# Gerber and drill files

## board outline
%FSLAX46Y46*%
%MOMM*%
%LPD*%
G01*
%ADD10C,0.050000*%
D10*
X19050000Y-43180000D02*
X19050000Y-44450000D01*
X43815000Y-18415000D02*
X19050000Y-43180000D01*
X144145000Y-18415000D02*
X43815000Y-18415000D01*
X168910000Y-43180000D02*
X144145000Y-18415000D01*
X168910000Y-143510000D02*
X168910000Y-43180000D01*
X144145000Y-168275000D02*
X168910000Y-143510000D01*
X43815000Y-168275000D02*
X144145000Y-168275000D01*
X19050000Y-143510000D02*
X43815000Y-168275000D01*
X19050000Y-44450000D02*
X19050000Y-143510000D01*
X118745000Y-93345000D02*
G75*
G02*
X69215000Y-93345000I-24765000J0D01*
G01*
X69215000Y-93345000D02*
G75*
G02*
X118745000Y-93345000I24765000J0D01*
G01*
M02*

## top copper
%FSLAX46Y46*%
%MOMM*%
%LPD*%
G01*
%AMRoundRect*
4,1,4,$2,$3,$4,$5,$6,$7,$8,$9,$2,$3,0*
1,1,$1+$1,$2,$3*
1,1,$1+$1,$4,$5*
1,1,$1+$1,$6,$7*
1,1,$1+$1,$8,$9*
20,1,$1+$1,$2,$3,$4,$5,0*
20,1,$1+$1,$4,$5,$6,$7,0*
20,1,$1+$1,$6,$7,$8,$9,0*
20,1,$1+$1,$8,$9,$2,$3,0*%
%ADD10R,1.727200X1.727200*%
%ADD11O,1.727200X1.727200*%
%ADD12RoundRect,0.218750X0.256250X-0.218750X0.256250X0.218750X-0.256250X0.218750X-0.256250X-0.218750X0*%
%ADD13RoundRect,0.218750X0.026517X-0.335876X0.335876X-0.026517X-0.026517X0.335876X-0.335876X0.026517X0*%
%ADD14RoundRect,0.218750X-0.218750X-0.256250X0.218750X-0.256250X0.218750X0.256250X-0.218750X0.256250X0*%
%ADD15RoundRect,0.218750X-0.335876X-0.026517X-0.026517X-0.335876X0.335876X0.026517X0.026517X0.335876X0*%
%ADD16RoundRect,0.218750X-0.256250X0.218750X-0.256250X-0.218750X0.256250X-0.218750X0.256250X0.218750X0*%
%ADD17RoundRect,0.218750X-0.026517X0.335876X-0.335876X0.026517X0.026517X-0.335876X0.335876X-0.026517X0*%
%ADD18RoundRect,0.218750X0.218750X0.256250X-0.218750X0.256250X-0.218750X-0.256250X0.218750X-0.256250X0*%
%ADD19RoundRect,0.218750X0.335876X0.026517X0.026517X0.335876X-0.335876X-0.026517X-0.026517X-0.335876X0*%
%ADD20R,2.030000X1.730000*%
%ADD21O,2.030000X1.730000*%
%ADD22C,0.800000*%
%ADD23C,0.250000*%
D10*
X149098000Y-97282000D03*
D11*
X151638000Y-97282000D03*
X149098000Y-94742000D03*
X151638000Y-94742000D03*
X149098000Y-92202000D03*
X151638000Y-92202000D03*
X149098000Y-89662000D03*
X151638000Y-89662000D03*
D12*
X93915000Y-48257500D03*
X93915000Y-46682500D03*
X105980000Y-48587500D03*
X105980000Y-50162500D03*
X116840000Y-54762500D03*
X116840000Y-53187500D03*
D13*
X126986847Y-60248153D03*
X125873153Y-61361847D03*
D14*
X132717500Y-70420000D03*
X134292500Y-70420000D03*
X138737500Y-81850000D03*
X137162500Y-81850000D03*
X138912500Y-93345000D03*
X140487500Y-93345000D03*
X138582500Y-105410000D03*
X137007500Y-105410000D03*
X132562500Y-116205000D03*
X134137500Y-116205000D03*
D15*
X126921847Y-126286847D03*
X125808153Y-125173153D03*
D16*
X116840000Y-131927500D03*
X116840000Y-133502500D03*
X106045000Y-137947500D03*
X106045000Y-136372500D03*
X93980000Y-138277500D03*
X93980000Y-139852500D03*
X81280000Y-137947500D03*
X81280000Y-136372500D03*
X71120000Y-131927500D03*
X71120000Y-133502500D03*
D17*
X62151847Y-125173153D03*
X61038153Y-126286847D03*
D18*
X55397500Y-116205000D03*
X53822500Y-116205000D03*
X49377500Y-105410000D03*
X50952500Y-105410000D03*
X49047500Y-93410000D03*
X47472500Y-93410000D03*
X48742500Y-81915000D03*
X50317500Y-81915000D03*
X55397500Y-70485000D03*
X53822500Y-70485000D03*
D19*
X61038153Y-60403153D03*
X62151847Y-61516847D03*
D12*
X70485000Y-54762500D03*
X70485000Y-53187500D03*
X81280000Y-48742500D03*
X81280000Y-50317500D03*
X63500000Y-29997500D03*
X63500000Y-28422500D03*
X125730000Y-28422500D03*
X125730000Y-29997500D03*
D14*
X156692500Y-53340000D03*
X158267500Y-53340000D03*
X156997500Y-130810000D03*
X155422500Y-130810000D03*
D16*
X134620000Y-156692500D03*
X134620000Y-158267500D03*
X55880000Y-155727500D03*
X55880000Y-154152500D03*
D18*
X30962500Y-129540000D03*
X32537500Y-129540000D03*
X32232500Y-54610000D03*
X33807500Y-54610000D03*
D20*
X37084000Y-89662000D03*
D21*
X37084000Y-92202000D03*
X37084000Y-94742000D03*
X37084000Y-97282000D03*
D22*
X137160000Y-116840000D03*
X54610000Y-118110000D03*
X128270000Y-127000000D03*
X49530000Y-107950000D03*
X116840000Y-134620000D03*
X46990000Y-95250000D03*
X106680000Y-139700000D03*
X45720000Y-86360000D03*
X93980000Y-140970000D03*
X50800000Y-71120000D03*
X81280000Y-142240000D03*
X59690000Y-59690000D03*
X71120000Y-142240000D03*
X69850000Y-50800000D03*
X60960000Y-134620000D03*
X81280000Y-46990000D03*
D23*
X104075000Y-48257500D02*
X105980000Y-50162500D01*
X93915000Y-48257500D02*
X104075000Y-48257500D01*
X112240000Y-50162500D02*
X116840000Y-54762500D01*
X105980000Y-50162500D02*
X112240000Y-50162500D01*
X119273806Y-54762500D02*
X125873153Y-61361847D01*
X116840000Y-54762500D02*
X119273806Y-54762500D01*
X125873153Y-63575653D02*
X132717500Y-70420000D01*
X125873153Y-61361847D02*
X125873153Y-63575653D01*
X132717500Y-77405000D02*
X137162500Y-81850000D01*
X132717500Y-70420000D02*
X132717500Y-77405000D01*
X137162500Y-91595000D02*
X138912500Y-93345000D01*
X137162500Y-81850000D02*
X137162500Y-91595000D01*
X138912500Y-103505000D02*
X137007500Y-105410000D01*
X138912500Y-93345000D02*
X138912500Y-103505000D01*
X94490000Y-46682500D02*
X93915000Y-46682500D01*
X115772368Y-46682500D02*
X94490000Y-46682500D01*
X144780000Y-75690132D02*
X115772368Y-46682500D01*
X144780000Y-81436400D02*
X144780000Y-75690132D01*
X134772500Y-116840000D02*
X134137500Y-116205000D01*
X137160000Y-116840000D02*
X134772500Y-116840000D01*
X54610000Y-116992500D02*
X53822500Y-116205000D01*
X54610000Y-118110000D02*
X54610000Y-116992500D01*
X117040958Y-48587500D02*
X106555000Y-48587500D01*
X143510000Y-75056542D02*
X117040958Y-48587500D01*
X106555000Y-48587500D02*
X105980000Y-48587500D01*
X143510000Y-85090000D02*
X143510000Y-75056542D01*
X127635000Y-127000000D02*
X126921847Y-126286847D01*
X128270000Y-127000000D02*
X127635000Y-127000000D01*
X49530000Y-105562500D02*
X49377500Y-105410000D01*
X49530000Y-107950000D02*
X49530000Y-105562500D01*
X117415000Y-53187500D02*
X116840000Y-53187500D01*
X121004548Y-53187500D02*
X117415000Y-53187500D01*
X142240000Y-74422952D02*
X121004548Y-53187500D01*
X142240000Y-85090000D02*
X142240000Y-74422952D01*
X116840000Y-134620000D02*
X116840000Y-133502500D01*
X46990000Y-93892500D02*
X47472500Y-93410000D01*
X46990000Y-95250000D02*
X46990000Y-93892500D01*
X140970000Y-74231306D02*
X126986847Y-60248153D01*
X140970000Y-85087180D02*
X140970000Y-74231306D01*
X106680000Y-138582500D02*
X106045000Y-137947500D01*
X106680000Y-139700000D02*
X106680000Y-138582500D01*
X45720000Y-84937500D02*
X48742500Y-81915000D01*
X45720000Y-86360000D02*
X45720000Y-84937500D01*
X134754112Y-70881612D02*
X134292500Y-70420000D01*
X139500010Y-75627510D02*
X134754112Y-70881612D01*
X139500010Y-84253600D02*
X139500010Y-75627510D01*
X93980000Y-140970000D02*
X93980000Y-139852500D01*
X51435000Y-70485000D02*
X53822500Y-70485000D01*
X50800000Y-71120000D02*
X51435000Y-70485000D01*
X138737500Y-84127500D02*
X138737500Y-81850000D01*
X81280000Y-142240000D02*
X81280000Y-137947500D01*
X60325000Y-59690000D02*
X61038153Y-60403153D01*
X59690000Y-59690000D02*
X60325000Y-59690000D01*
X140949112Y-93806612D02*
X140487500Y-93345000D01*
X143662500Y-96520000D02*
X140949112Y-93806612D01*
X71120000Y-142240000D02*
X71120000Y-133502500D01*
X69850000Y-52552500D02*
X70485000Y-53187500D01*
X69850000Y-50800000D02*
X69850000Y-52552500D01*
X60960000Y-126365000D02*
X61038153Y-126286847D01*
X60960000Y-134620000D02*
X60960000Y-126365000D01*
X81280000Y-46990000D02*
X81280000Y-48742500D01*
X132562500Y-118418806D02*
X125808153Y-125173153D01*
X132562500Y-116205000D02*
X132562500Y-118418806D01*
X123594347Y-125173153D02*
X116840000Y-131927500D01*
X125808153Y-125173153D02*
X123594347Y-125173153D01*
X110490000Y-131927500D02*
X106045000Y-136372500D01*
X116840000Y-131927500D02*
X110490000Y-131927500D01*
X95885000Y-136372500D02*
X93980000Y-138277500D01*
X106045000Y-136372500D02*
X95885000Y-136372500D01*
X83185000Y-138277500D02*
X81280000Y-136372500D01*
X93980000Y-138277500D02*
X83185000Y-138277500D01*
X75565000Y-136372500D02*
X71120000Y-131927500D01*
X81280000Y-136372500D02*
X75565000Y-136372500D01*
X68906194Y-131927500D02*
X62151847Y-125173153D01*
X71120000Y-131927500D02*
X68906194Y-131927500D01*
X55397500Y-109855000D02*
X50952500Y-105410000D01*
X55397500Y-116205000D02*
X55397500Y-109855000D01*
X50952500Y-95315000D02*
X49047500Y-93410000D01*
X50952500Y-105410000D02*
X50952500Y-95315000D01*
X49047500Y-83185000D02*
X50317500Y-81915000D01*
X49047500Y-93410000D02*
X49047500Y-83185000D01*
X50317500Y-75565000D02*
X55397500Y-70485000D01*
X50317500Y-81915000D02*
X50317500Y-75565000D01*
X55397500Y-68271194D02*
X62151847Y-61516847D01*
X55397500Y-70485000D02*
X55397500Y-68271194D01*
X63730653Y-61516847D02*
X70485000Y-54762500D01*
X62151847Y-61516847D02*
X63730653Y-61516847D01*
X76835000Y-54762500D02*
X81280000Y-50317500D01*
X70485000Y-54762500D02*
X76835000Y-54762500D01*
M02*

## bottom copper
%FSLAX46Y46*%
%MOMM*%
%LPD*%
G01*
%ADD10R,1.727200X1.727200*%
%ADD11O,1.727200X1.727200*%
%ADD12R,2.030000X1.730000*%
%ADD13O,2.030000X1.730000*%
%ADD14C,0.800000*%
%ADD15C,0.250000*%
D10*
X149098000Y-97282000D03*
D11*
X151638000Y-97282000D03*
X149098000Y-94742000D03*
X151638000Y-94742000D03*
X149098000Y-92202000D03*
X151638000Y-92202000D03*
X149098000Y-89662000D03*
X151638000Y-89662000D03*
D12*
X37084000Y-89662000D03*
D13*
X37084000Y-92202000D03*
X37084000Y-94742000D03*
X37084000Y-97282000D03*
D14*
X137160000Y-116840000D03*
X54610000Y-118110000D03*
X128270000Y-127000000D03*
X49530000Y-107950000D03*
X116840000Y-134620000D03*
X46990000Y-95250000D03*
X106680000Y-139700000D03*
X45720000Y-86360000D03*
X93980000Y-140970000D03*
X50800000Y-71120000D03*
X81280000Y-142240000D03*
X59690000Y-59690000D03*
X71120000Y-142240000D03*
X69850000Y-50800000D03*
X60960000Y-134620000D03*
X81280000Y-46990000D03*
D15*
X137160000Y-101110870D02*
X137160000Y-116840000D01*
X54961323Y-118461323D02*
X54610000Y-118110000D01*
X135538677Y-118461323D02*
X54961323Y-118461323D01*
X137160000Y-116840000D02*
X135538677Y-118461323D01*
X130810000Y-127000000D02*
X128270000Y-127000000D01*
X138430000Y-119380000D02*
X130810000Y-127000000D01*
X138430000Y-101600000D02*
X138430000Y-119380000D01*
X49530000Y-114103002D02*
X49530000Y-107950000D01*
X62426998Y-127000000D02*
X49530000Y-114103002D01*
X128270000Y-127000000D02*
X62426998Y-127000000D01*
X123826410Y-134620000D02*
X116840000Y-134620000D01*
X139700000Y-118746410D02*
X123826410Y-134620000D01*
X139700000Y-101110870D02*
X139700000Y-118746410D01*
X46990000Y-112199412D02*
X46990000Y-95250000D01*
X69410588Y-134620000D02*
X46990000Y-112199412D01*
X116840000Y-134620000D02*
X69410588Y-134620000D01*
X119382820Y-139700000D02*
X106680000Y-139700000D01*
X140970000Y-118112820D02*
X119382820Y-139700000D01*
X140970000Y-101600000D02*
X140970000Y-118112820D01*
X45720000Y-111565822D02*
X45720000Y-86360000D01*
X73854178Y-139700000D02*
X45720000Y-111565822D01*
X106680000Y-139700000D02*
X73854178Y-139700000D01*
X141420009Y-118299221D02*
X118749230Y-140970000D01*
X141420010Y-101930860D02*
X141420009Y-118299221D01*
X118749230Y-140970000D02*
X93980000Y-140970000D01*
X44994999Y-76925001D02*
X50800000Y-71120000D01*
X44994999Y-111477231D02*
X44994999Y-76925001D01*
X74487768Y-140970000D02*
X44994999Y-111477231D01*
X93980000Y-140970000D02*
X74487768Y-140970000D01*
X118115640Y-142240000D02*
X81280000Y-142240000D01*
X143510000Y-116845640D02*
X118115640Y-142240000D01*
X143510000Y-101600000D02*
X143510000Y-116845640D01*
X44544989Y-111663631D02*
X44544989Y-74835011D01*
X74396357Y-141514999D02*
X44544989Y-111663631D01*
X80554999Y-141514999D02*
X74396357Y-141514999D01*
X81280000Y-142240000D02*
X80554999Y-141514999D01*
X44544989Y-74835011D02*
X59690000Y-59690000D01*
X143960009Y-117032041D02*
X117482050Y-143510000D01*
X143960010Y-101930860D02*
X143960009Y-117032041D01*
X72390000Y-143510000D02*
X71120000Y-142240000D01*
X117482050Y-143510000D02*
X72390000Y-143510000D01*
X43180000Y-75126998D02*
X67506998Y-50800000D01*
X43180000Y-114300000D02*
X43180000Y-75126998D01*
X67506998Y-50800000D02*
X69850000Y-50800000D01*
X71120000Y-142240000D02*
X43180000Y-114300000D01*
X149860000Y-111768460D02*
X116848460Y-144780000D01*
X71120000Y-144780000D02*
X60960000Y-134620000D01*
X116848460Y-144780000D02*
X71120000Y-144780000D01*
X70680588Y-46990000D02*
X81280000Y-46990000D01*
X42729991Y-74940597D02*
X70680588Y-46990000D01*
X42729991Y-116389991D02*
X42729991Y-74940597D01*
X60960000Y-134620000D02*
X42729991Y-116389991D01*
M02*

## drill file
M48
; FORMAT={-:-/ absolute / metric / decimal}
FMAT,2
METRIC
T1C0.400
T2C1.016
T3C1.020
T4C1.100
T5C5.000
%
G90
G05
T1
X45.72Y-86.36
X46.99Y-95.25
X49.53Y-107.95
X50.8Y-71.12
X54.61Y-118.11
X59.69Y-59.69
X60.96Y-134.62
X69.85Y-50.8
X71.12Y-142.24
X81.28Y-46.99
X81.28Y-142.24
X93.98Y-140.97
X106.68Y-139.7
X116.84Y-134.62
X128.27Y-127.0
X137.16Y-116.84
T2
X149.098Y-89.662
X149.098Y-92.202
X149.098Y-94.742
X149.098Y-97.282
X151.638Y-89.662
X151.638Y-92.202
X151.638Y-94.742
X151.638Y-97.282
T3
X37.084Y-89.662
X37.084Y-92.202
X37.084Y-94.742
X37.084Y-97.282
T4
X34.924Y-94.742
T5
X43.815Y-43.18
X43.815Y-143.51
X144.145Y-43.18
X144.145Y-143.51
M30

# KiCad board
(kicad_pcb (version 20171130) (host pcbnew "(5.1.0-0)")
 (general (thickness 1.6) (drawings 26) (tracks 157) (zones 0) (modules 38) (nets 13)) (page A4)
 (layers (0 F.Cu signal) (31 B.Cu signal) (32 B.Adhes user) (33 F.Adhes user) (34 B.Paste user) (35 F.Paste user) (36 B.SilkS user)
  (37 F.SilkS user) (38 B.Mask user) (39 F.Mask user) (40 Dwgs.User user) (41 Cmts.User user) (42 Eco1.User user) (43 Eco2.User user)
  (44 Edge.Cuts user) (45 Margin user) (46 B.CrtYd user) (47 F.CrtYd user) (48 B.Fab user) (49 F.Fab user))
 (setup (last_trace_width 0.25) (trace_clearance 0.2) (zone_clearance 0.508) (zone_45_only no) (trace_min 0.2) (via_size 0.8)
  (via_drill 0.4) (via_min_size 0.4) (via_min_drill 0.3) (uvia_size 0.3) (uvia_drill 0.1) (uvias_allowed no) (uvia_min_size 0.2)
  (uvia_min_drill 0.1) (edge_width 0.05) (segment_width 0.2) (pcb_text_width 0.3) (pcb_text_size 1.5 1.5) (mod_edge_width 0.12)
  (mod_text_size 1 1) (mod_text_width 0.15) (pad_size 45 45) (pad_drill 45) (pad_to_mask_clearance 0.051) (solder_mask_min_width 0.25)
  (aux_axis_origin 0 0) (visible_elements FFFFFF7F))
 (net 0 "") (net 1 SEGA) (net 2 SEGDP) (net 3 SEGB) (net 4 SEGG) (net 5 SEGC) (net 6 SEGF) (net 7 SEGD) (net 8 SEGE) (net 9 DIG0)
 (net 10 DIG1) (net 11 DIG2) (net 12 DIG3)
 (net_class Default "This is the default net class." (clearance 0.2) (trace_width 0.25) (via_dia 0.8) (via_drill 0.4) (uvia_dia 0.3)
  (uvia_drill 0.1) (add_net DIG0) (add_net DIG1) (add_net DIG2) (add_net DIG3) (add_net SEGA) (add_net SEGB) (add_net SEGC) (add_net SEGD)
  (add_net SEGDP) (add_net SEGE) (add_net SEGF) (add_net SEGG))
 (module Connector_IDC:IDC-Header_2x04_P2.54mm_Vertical (layer B.Cu) (at 149.098 97.282)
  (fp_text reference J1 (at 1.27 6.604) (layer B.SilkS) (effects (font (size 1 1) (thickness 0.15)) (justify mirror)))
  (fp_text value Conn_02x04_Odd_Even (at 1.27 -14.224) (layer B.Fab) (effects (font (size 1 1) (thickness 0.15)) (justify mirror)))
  (pad 1 thru_hole rect (at 0 0) (size 1.7272 1.7272) (drill 1.016) (layers *.Cu *.Mask) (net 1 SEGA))
  (pad 2 thru_hole oval (at 2.54 0) (size 1.7272 1.7272) (drill 1.016) (layers *.Cu *.Mask) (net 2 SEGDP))
  (pad 3 thru_hole oval (at 0 -2.54) (size 1.7272 1.7272) (drill 1.016) (layers *.Cu *.Mask) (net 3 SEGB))
  (pad 4 thru_hole oval (at 2.54 -2.54) (size 1.7272 1.7272) (drill 1.016) (layers *.Cu *.Mask) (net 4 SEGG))
  (pad 5 thru_hole oval (at 0 -5.08) (size 1.7272 1.7272) (drill 1.016) (layers *.Cu *.Mask) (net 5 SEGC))
  (pad 6 thru_hole oval (at 2.54 -5.08) (size 1.7272 1.7272) (drill 1.016) (layers *.Cu *.Mask) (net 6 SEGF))
  (pad 7 thru_hole oval (at 0 -7.62) (size 1.7272 1.7272) (drill 1.016) (layers *.Cu *.Mask) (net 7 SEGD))
  (pad 8 thru_hole oval (at 2.54 -7.62) (size 1.7272 1.7272) (drill 1.016) (layers *.Cu *.Mask) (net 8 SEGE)))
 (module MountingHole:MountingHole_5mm (layer F.Cu) (at 144.145 43.18)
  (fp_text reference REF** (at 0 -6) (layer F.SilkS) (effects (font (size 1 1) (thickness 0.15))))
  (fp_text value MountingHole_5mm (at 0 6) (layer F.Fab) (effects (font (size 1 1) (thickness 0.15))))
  (pad 1 np_thru_hole circle (at 0 0) (size 5 5) (drill 5) (layers *.Cu *.Mask)))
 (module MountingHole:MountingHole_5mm (layer F.Cu) (at 43.815 43.18)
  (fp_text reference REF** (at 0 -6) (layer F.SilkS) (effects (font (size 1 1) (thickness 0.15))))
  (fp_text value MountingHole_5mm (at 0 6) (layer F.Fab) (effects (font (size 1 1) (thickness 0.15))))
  (pad 1 np_thru_hole circle (at 0 0) (size 5 5) (drill 5) (layers *.Cu *.Mask)))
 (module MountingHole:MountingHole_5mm (layer F.Cu) (at 43.815 143.51)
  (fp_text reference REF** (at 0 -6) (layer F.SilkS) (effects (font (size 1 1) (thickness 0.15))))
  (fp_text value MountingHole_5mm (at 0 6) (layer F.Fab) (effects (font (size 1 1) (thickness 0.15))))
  (pad 1 np_thru_hole circle (at 0 0) (size 5 5) (drill 5) (layers *.Cu *.Mask)))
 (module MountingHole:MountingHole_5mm (layer F.Cu) (at 144.145 143.51)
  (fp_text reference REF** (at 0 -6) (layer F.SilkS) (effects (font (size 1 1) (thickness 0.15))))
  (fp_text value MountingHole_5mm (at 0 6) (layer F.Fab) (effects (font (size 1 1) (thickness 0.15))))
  (pad 1 np_thru_hole circle (at 0 0) (size 5 5) (drill 5) (layers *.Cu *.Mask)))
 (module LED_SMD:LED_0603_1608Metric (layer F.Cu) (at 93.915 47.47 90)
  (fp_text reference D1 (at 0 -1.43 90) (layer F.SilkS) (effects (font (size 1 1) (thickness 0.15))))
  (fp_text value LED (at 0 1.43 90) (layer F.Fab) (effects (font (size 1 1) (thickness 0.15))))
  (pad 1 smd roundrect (at -0.7875 0 90) (size 0.875 0.95) (layers F.Cu F.Paste F.Mask) (roundrect_rratio 0.25) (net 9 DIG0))
  (pad 2 smd roundrect (at 0.7875 0 90) (size 0.875 0.95) (layers F.Cu F.Paste F.Mask) (roundrect_rratio 0.25) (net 1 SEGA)))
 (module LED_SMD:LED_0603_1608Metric (layer F.Cu) (at 105.98 49.375 90)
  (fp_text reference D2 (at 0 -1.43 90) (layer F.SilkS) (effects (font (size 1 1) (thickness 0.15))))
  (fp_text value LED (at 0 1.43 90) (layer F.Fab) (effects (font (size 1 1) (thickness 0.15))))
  (pad 2 smd roundrect (at 0.7875 0 90) (size 0.875 0.95) (layers F.Cu F.Paste F.Mask) (roundrect_rratio 0.25) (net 3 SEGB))
  (pad 1 smd roundrect (at -0.7875 0 90) (size 0.875 0.95) (layers F.Cu F.Paste F.Mask) (roundrect_rratio 0.25) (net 9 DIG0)))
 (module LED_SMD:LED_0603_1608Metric (layer F.Cu) (at 116.84 53.975 90)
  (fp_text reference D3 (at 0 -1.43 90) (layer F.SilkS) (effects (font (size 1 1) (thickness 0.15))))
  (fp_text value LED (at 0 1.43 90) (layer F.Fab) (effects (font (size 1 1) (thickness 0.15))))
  (pad 1 smd roundrect (at -0.7875 0 90) (size 0.875 0.95) (layers F.Cu F.Paste F.Mask) (roundrect_rratio 0.25) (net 9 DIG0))
  (pad 2 smd roundrect (at 0.7875 0 90) (size 0.875 0.95) (layers F.Cu F.Paste F.Mask) (roundrect_rratio 0.25) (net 5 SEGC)))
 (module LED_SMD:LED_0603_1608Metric (layer F.Cu) (at 126.43 60.805 45)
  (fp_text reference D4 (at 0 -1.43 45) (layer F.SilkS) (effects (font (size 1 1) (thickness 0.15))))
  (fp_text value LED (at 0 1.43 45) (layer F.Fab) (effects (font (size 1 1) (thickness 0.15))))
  (pad 2 smd roundrect (at 0.7875 0 45) (size 0.875 0.95) (layers F.Cu F.Paste F.Mask) (roundrect_rratio 0.25) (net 7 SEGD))
  (pad 1 smd roundrect (at -0.7875 0 45) (size 0.875 0.95) (layers F.Cu F.Paste F.Mask) (roundrect_rratio 0.25) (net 9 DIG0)))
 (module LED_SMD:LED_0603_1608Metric (layer F.Cu) (at 133.505 70.42)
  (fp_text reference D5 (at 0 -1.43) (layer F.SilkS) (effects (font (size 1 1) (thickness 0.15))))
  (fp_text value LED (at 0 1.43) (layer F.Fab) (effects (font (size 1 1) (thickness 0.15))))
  (pad 1 smd roundrect (at -0.7875 0) (size 0.875 0.95) (layers F.Cu F.Paste F.Mask) (roundrect_rratio 0.25) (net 9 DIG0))
  (pad 2 smd roundrect (at 0.7875 0) (size 0.875 0.95) (layers F.Cu F.Paste F.Mask) (roundrect_rratio 0.25) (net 8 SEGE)))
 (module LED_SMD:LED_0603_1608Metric (layer F.Cu) (at 137.95 81.85)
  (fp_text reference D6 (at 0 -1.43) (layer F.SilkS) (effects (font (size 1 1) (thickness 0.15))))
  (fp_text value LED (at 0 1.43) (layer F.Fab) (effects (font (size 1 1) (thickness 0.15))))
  (pad 2 smd roundrect (at 0.7875 0) (size 0.875 0.95) (layers F.Cu F.Paste F.Mask) (roundrect_rratio 0.25) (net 6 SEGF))
  (pad 1 smd roundrect (at -0.7875 0) (size 0.875 0.95) (layers F.Cu F.Paste F.Mask) (roundrect_rratio 0.25) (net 9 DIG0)))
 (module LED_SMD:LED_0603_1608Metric (layer F.Cu) (at 139.7 93.345)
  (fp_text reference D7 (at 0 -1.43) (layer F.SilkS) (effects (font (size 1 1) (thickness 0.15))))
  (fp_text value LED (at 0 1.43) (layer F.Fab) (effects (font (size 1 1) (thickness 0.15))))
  (pad 1 smd roundrect (at -0.7875 0) (size 0.875 0.95) (layers F.Cu F.Paste F.Mask) (roundrect_rratio 0.25) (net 9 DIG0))
  (pad 2 smd roundrect (at 0.7875 0) (size 0.875 0.95) (layers F.Cu F.Paste F.Mask) (roundrect_rratio 0.25) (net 4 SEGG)))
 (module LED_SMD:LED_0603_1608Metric (layer F.Cu) (at 137.795 105.41)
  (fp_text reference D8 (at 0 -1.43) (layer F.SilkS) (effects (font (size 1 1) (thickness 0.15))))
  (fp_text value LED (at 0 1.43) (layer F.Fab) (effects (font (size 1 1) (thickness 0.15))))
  (pad 2 smd roundrect (at 0.7875 0) (size 0.875 0.95) (layers F.Cu F.Paste F.Mask) (roundrect_rratio 0.25) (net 2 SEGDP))
  (pad 1 smd roundrect (at -0.7875 0) (size 0.875 0.95) (layers F.Cu F.Paste F.Mask) (roundrect_rratio 0.25) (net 9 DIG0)))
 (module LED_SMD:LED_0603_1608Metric (layer F.Cu) (at 133.35 116.205)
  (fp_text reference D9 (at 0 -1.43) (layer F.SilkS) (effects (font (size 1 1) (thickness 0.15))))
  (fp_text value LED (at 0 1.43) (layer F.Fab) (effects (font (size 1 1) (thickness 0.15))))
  (pad 1 smd roundrect (at -0.7875 0) (size 0.875 0.95) (layers F.Cu F.Paste F.Mask) (roundrect_rratio 0.25) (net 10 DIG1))
  (pad 2 smd roundrect (at 0.7875 0) (size 0.875 0.95) (layers F.Cu F.Paste F.Mask) (roundrect_rratio 0.25) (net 1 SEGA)))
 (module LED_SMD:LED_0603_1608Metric (layer F.Cu) (at 126.365 125.73 315)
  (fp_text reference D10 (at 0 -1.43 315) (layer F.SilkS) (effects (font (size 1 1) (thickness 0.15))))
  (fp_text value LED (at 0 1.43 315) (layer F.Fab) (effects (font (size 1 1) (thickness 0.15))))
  (pad 2 smd roundrect (at 0.7875 0 315) (size 0.875 0.95) (layers F.Cu F.Paste F.Mask) (roundrect_rratio 0.25) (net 3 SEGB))
  (pad 1 smd roundrect (at -0.7875 0 315) (size 0.875 0.95) (layers F.Cu F.Paste F.Mask) (roundrect_rratio 0.25) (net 10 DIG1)))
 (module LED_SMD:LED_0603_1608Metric (layer F.Cu) (at 116.84 132.715 270)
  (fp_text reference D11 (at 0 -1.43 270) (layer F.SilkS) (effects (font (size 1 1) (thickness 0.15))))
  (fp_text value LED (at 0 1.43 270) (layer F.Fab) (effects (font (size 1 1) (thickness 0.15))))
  (pad 1 smd roundrect (at -0.7875 0 270) (size 0.875 0.95) (layers F.Cu F.Paste F.Mask) (roundrect_rratio 0.25) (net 10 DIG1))
  (pad 2 smd roundrect (at 0.7875 0 270) (size 0.875 0.95) (layers F.Cu F.Paste F.Mask) (roundrect_rratio 0.25) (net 5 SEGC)))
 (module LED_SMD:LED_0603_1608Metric (layer F.Cu) (at 106.045 137.16 270)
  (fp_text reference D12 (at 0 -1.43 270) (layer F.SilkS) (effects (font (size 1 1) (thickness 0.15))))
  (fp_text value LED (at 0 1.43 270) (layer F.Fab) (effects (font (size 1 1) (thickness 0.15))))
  (pad 2 smd roundrect (at 0.7875 0 270) (size 0.875 0.95) (layers F.Cu F.Paste F.Mask) (roundrect_rratio 0.25) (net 7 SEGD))
  (pad 1 smd roundrect (at -0.7875 0 270) (size 0.875 0.95) (layers F.Cu F.Paste F.Mask) (roundrect_rratio 0.25) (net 10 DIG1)))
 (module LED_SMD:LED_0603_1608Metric (layer F.Cu) (at 93.98 139.065 270)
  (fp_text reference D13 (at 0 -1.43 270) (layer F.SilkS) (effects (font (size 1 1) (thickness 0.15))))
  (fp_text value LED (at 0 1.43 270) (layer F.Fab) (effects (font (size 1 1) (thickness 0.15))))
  (pad 1 smd roundrect (at -0.7875 0 270) (size 0.875 0.95) (layers F.Cu F.Paste F.Mask) (roundrect_rratio 0.25) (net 10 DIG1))
  (pad 2 smd roundrect (at 0.7875 0 270) (size 0.875 0.95) (layers F.Cu F.Paste F.Mask) (roundrect_rratio 0.25) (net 8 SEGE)))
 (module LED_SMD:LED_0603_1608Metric (layer F.Cu) (at 81.28 137.16 270)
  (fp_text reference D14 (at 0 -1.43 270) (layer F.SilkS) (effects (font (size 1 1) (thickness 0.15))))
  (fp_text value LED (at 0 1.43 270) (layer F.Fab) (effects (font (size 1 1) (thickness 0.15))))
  (pad 2 smd roundrect (at 0.7875 0 270) (size 0.875 0.95) (layers F.Cu F.Paste F.Mask) (roundrect_rratio 0.25) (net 6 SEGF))
  (pad 1 smd roundrect (at -0.7875 0 270) (size 0.875 0.95) (layers F.Cu F.Paste F.Mask) (roundrect_rratio 0.25) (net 10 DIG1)))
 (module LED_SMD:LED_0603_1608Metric (layer F.Cu) (at 71.12 132.715 270)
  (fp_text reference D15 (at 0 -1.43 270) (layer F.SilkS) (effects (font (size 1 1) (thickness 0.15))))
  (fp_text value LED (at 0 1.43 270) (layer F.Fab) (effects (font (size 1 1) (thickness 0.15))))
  (pad 1 smd roundrect (at -0.7875 0 270) (size 0.875 0.95) (layers F.Cu F.Paste F.Mask) (roundrect_rratio 0.25) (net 10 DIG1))
  (pad 2 smd roundrect (at 0.7875 0 270) (size 0.875 0.95) (layers F.Cu F.Paste F.Mask) (roundrect_rratio 0.25) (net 4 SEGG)))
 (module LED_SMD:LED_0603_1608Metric (layer F.Cu) (at 61.595 125.73 225)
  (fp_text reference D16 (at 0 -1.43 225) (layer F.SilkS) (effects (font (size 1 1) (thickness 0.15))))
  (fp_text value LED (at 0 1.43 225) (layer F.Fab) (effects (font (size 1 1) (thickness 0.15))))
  (pad 1 smd roundrect (at -0.7875 0 225) (size 0.875 0.95) (layers F.Cu F.Paste F.Mask) (roundrect_rratio 0.25) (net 10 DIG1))
  (pad 2 smd roundrect (at 0.7875 0 225) (size 0.875 0.95) (layers F.Cu F.Paste F.Mask) (roundrect_rratio 0.25) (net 2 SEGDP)))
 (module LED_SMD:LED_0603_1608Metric (layer F.Cu) (at 54.61 116.205 180)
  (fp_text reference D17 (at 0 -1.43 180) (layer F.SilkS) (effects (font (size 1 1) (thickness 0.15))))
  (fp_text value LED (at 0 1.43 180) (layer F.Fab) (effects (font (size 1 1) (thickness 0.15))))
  (pad 1 smd roundrect (at -0.7875 0 180) (size 0.875 0.95) (layers F.Cu F.Paste F.Mask) (roundrect_rratio 0.25) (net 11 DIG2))
  (pad 2 smd roundrect (at 0.7875 0 180) (size 0.875 0.95) (layers F.Cu F.Paste F.Mask) (roundrect_rratio 0.25) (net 1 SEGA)))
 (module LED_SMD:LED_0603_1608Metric (layer F.Cu) (at 50.165 105.41 180)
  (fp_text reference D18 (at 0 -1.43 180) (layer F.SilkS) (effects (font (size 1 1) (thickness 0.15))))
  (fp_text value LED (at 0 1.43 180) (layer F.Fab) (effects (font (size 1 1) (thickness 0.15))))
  (pad 2 smd roundrect (at 0.7875 0 180) (size 0.875 0.95) (layers F.Cu F.Paste F.Mask) (roundrect_rratio 0.25) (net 3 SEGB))
  (pad 1 smd roundrect (at -0.7875 0 180) (size 0.875 0.95) (layers F.Cu F.Paste F.Mask) (roundrect_rratio 0.25) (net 11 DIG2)))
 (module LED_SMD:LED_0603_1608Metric (layer F.Cu) (at 48.26 93.41 180)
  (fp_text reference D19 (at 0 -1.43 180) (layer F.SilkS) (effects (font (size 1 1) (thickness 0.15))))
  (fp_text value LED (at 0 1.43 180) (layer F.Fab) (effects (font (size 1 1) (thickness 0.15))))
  (pad 1 smd roundrect (at -0.7875 0 180) (size 0.875 0.95) (layers F.Cu F.Paste F.Mask) (roundrect_rratio 0.25) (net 11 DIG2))
  (pad 2 smd roundrect (at 0.7875 0 180) (size 0.875 0.95) (layers F.Cu F.Paste F.Mask) (roundrect_rratio 0.25) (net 5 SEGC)))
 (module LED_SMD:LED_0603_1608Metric (layer F.Cu) (at 49.53 81.915 180)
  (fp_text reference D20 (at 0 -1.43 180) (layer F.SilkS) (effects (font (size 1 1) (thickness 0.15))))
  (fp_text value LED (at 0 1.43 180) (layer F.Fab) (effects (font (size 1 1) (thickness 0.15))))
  (pad 2 smd roundrect (at 0.7875 0 180) (size 0.875 0.95) (layers F.Cu F.Paste F.Mask) (roundrect_rratio 0.25) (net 7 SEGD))
  (pad 1 smd roundrect (at -0.7875 0 180) (size 0.875 0.95) (layers F.Cu F.Paste F.Mask) (roundrect_rratio 0.25) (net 11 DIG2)))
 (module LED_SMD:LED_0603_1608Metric (layer F.Cu) (at 54.61 70.485 180)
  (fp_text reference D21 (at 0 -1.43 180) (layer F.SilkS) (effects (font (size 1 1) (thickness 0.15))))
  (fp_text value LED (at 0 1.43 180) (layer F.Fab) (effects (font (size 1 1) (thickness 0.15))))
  (pad 1 smd roundrect (at -0.7875 0 180) (size 0.875 0.95) (layers F.Cu F.Paste F.Mask) (roundrect_rratio 0.25) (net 11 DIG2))
  (pad 2 smd roundrect (at 0.7875 0 180) (size 0.875 0.95) (layers F.Cu F.Paste F.Mask) (roundrect_rratio 0.25) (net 8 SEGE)))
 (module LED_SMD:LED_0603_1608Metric (layer F.Cu) (at 61.595 60.96 135)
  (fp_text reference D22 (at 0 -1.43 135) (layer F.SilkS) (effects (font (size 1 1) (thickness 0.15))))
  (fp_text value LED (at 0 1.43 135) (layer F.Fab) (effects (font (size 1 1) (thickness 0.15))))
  (pad 2 smd roundrect (at 0.7875 0 135) (size 0.875 0.95) (layers F.Cu F.Paste F.Mask) (roundrect_rratio 0.25) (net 6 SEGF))
  (pad 1 smd roundrect (at -0.7875 0 135) (size 0.875 0.95) (layers F.Cu F.Paste F.Mask) (roundrect_rratio 0.25) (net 11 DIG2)))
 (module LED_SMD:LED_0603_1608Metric (layer F.Cu) (at 70.485 53.975 90)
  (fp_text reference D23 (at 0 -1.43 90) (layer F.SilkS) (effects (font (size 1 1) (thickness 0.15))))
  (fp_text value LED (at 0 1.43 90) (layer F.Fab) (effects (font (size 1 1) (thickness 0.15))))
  (pad 1 smd roundrect (at -0.7875 0 90) (size 0.875 0.95) (layers F.Cu F.Paste F.Mask) (roundrect_rratio 0.25) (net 11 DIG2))
  (pad 2 smd roundrect (at 0.7875 0 90) (size 0.875 0.95) (layers F.Cu F.Paste F.Mask) (roundrect_rratio 0.25) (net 4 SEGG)))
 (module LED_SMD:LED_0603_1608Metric (layer F.Cu) (at 81.28 49.53 90)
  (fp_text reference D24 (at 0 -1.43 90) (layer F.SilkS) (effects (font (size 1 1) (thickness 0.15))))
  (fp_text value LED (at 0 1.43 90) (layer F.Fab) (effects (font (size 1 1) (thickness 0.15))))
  (pad 2 smd roundrect (at 0.7875 0 90) (size 0.875 0.95) (layers F.Cu F.Paste F.Mask) (roundrect_rratio 0.25) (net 2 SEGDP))
  (pad 1 smd roundrect (at -0.7875 0 90) (size 0.875 0.95) (layers F.Cu F.Paste F.Mask) (roundrect_rratio 0.25) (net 11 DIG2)))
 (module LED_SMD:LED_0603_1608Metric (layer F.Cu) (at 63.5 29.21 90)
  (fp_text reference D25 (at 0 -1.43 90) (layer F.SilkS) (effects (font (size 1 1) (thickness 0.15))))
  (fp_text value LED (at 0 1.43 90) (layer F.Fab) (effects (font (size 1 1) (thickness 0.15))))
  (pad 1 smd roundrect (at -0.7875 0 90) (size 0.875 0.95) (layers F.Cu F.Paste F.Mask) (roundrect_rratio 0.25) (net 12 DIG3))
  (pad 2 smd roundrect (at 0.7875 0 90) (size 0.875 0.95) (layers F.Cu F.Paste F.Mask) (roundrect_rratio 0.25) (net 1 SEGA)))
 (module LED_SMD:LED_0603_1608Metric (layer F.Cu) (at 125.73 29.21 90)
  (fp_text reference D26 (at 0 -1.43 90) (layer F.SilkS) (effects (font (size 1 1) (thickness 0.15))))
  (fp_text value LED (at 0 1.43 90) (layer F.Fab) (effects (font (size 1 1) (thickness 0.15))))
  (pad 2 smd roundrect (at 0.7875 0 90) (size 0.875 0.95) (layers F.Cu F.Paste F.Mask) (roundrect_rratio 0.25) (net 3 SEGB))
  (pad 1 smd roundrect (at -0.7875 0 90) (size 0.875 0.95) (layers F.Cu F.Paste F.Mask) (roundrect_rratio 0.25) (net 12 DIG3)))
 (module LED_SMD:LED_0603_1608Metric (layer F.Cu) (at 157.48 53.34)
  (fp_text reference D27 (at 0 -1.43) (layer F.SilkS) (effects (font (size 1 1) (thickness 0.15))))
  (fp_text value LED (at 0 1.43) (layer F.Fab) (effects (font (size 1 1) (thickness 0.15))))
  (pad 1 smd roundrect (at -0.7875 0) (size 0.875 0.95) (layers F.Cu F.Paste F.Mask) (roundrect_rratio 0.25) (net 12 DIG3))
  (pad 2 smd roundrect (at 0.7875 0) (size 0.875 0.95) (layers F.Cu F.Paste F.Mask) (roundrect_rratio 0.25) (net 5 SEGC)))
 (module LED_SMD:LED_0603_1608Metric (layer F.Cu) (at 156.21 130.81)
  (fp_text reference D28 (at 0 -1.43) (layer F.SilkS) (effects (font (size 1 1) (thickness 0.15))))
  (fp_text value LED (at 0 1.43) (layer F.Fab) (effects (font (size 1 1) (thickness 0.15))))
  (pad 2 smd roundrect (at 0.7875 0) (size 0.875 0.95) (layers F.Cu F.Paste F.Mask) (roundrect_rratio 0.25) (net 7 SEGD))
  (pad 1 smd roundrect (at -0.7875 0) (size 0.875 0.95) (layers F.Cu F.Paste F.Mask) (roundrect_rratio 0.25) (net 12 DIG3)))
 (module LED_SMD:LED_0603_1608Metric (layer F.Cu) (at 134.62 157.48 270)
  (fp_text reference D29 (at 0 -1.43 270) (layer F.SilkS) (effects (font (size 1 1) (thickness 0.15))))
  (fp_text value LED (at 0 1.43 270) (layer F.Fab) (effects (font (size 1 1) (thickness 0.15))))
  (pad 1 smd roundrect (at -0.7875 0 270) (size 0.875 0.95) (layers F.Cu F.Paste F.Mask) (roundrect_rratio 0.25) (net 12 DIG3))
  (pad 2 smd roundrect (at 0.7875 0 270) (size 0.875 0.95) (layers F.Cu F.Paste F.Mask) (roundrect_rratio 0.25) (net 8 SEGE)))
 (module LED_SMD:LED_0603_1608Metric (layer F.Cu) (at 55.88 154.94 270)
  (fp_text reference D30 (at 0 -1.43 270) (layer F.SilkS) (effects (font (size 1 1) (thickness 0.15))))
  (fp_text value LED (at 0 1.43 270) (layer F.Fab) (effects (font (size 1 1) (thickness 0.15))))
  (pad 2 smd roundrect (at 0.7875 0 270) (size 0.875 0.95) (layers F.Cu F.Paste F.Mask) (roundrect_rratio 0.25) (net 6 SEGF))
  (pad 1 smd roundrect (at -0.7875 0 270) (size 0.875 0.95) (layers F.Cu F.Paste F.Mask) (roundrect_rratio 0.25) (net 12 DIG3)))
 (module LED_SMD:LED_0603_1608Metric (layer F.Cu) (at 31.75 129.54 180)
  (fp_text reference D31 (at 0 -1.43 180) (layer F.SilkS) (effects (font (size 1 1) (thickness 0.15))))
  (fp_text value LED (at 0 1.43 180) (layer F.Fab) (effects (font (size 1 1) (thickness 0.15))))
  (pad 2 smd roundrect (at 0.7875 0 180) (size 0.875 0.95) (layers F.Cu F.Paste F.Mask) (roundrect_rratio 0.25) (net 4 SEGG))
  (pad 1 smd roundrect (at -0.7875 0 180) (size 0.875 0.95) (layers F.Cu F.Paste F.Mask) (roundrect_rratio 0.25) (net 12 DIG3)))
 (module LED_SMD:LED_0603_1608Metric (layer F.Cu) (at 33.02 54.61 180)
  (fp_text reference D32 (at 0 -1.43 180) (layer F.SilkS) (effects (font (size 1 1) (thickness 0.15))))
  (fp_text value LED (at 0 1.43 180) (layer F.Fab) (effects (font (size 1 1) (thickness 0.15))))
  (pad 2 smd roundrect (at 0.7875 0 180) (size 0.875 0.95) (layers F.Cu F.Paste F.Mask) (roundrect_rratio 0.25) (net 2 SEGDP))
  (pad 1 smd roundrect (at -0.7875 0 180) (size 0.875 0.95) (layers F.Cu F.Paste F.Mask) (roundrect_rratio 0.25) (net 12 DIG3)))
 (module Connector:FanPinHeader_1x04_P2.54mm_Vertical (layer B.Cu) (at 37.084 89.662 270)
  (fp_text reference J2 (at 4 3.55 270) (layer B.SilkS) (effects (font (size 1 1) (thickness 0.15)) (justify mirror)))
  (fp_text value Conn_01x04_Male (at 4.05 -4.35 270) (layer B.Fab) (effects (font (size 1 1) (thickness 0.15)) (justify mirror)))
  (pad 1 thru_hole rect (at 0 0 180) (size 2.03 1.73) (drill 1.02) (layers *.Cu *.Mask) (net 9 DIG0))
  (pad 2 thru_hole oval (at 2.54 0 180) (size 2.03 1.73) (drill 1.02) (layers *.Cu *.Mask) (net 10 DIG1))
  (pad 3 thru_hole oval (at 5.08 0 180) (size 2.03 1.73) (drill 1.02) (layers *.Cu *.Mask) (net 11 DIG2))
  (pad 4 thru_hole oval (at 7.62 0 180) (size 2.03 1.73) (drill 1.02) (layers *.Cu *.Mask) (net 12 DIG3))
  (pad "" np_thru_hole circle (at 5.08 2.16 180) (size 1.1 1.1) (drill 1.1) (layers *.Cu *.Mask)))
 (gr_line (start 19.05 43.18) (end 19.05 44.45) (layer Edge.Cuts) (width 0.05))
 (gr_line (start 43.815 18.415) (end 19.05 43.18) (layer Edge.Cuts) (width 0.05))
 (gr_line (start 144.145 18.415) (end 43.815 18.415) (layer Edge.Cuts) (width 0.05))
 (gr_line (start 168.91 43.18) (end 144.145 18.415) (layer Edge.Cuts) (width 0.05))
 (gr_line (start 168.91 143.51) (end 168.91 43.18) (layer Edge.Cuts) (width 0.05))
 (gr_line (start 144.145 168.275) (end 168.91 143.51) (layer Edge.Cuts) (width 0.05))
 (gr_line (start 43.815 168.275) (end 144.145 168.275) (layer Edge.Cuts) (width 0.05))
 (gr_line (start 19.05 143.51) (end 43.815 168.275) (layer Edge.Cuts) (width 0.05))
 (gr_line (start 19.05 44.45) (end 19.05 143.51) (layer Edge.Cuts) (width 0.05))
 (gr_circle (center 93.98 93.345) (end 118.745 93.345) (layer Edge.Cuts) (width 0.05))
 (segment (start 104.075 48.2575) (end 105.98 50.1625) (width 0.25) (layer F.Cu) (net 9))
 (segment (start 93.915 48.2575) (end 104.075 48.2575) (width 0.25) (layer F.Cu) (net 9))
 (segment (start 112.24 50.1625) (end 116.84 54.7625) (width 0.25) (layer F.Cu) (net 9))
 (segment (start 105.98 50.1625) (end 112.24 50.1625) (width 0.25) (layer F.Cu) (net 9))
 (segment (start 119.273806 54.7625) (end 125.873153 61.361847) (width 0.25) (layer F.Cu) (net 9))
 (segment (start 116.84 54.7625) (end 119.273806 54.7625) (width 0.25) (layer F.Cu) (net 9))
 (segment (start 125.873153 63.575653) (end 132.7175 70.42) (width 0.25) (layer F.Cu) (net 9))
 (segment (start 125.873153 61.361847) (end 125.873153 63.575653) (width 0.25) (layer F.Cu) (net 9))
 (segment (start 132.7175 77.405) (end 137.1625 81.85) (width 0.25) (layer F.Cu) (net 9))
 (segment (start 132.7175 70.42) (end 132.7175 77.405) (width 0.25) (layer F.Cu) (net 9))
 (segment (start 137.1625 91.595) (end 138.9125 93.345) (width 0.25) (layer F.Cu) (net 9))
 (segment (start 137.1625 81.85) (end 137.1625 91.595) (width 0.25) (layer F.Cu) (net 9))
 (segment (start 138.9125 103.505) (end 137.0075 105.41) (width 0.25) (layer F.Cu) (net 9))
 (segment (start 138.9125 93.345) (end 138.9125 103.505) (width 0.25) (layer F.Cu) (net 9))
 (segment (start 94.49 46.6825) (end 93.915 46.6825) (width 0.25) (layer F.Cu) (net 1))
 (segment (start 115.772368 46.6825) (end 94.49 46.6825) (width 0.25) (layer F.Cu) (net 1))
 (segment (start 144.78 75.690132) (end 115.772368 46.6825) (width 0.25) (layer F.Cu) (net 1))
 (segment (start 144.78 81.4364) (end 144.78 75.690132) (width 0.25) (layer F.Cu) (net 1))
 (via (at 137.16 116.84) (size 0.8) (drill 0.4) (layers F.Cu B.Cu) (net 1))
 (segment (start 137.16 101.11087) (end 137.16 116.84) (width 0.25) (layer B.Cu) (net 1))
 (segment (start 134.7725 116.84) (end 134.1375 116.205) (width 0.25) (layer F.Cu) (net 1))
 (segment (start 137.16 116.84) (end 134.7725 116.84) (width 0.25) (layer F.Cu) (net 1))
 (via (at 54.61 118.11) (size 0.8) (drill 0.4) (layers F.Cu B.Cu) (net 1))
 (segment (start 54.961323 118.461323) (end 54.61 118.11) (width 0.25) (layer B.Cu) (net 1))
 (segment (start 135.538677 118.461323) (end 54.961323 118.461323) (width 0.25) (layer B.Cu) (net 1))
 (segment (start 137.16 116.84) (end 135.538677 118.461323) (width 0.25) (layer B.Cu) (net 1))
 (segment (start 54.61 116.9925) (end 53.8225 116.205) (width 0.25) (layer F.Cu) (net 1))
 (segment (start 54.61 118.11) (end 54.61 116.9925) (width 0.25) (layer F.Cu) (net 1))
 (segment (start 117.040958 48.5875) (end 106.555 48.5875) (width 0.25) (layer F.Cu) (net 3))
 (segment (start 143.51 75.056542) (end 117.040958 48.5875) (width 0.25) (layer F.Cu) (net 3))
 (segment (start 106.555 48.5875) (end 105.98 48.5875) (width 0.25) (layer F.Cu) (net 3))
 (segment (start 143.51 85.09) (end 143.51 75.056542) (width 0.25) (layer F.Cu) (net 3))
 (via (at 128.27 127) (size 0.8) (drill 0.4) (layers F.Cu B.Cu) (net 3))
 (segment (start 130.81 127) (end 128.27 127) (width 0.25) (layer B.Cu) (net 3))
 (segment (start 138.43 119.38) (end 130.81 127) (width 0.25) (layer B.Cu) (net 3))
 (segment (start 138.43 101.6) (end 138.43 119.38) (width 0.25) (layer B.Cu) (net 3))
 (segment (start 127.635 127) (end 126.921847 126.286847) (width 0.25) (layer F.Cu) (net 3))
 (segment (start 128.27 127) (end 127.635 127) (width 0.25) (layer F.Cu) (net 3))
 (segment (start 49.53 114.103002) (end 49.53 107.95) (width 0.25) (layer B.Cu) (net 3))
 (segment (start 62.426998 127) (end 49.53 114.103002) (width 0.25) (layer B.Cu) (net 3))
 (via (at 49.53 107.95) (size 0.8) (drill 0.4) (layers F.Cu B.Cu) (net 3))
 (segment (start 128.27 127) (end 62.426998 127) (width 0.25) (layer B.Cu) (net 3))
 (segment (start 49.53 105.5625) (end 49.3775 105.41) (width 0.25) (layer F.Cu) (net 3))
 (segment (start 49.53 107.95) (end 49.53 105.5625) (width 0.25) (layer F.Cu) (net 3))
 (segment (start 117.415 53.1875) (end 116.84 53.1875) (width 0.25) (layer F.Cu) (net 5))
 (segment (start 121.004548 53.1875) (end 117.415 53.1875) (width 0.25) (layer F.Cu) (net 5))
 (segment (start 142.24 74.422952) (end 121.004548 53.1875) (width 0.25) (layer F.Cu) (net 5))
 (segment (start 142.24 85.09) (end 142.24 74.422952) (width 0.25) (layer F.Cu) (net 5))
 (via (at 116.84 134.62) (size 0.8) (drill 0.4) (layers F.Cu B.Cu) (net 5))
 (segment (start 123.82641 134.62) (end 116.84 134.62) (width 0.25) (layer B.Cu) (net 5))
 (segment (start 139.7 118.74641) (end 123.82641 134.62) (width 0.25) (layer B.Cu) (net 5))
 (segment (start 139.7 101.11087) (end 139.7 118.74641) (width 0.25) (layer B.Cu) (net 5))
 (segment (start 116.84 134.62) (end 116.84 133.5025) (width 0.25) (layer F.Cu) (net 5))
 (via (at 46.99 95.25) (size 0.8) (drill 0.4) (layers F.Cu B.Cu) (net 5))
 (segment (start 46.99 112.199412) (end 46.99 95.25) (width 0.25) (layer B.Cu) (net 5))
 (segment (start 69.410588 134.62) (end 46.99 112.199412) (width 0.25) (layer B.Cu) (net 5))
 (segment (start 116.84 134.62) (end 69.410588 134.62) (width 0.25) (layer B.Cu) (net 5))
 (segment (start 46.99 93.8925) (end 47.4725 93.41) (width 0.25) (layer F.Cu) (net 5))
 (segment (start 46.99 95.25) (end 46.99 93.8925) (width 0.25) (layer F.Cu) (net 5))
 (segment (start 140.97 74.231306) (end 126.986847 60.248153) (width 0.25) (layer F.Cu) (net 7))
 (segment (start 140.97 85.08718) (end 140.97 74.231306) (width 0.25) (layer F.Cu) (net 7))
 (via (at 106.68 139.7) (size 0.8) (drill 0.4) (layers F.Cu B.Cu) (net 7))
 (segment (start 119.38282 139.7) (end 106.68 139.7) (width 0.25) (layer B.Cu) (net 7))
 (segment (start 140.97 118.11282) (end 119.38282 139.7) (width 0.25) (layer B.Cu) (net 7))
 (segment (start 140.97 101.6) (end 140.97 118.11282) (width 0.25) (layer B.Cu) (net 7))
 (segment (start 106.68 138.5825) (end 106.045 137.9475) (width 0.25) (layer F.Cu) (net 7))
 (segment (start 106.68 139.7) (end 106.68 138.5825) (width 0.25) (layer F.Cu) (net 7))
 (via (at 45.72 86.36) (size 0.8) (drill 0.4) (layers F.Cu B.Cu) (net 7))
 (segment (start 45.72 111.565822) (end 45.72 86.36) (width 0.25) (layer B.Cu) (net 7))
 (segment (start 73.854178 139.7) (end 45.72 111.565822) (width 0.25) (layer B.Cu) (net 7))
 (segment (start 106.68 139.7) (end 73.854178 139.7) (width 0.25) (layer B.Cu) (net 7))
 (segment (start 45.72 84.9375) (end 48.7425 81.915) (width 0.25) (layer F.Cu) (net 7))
 (segment (start 45.72 86.36) (end 45.72 84.9375) (width 0.25) (layer F.Cu) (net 7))
 (segment (start 134.754112 70.881612) (end 134.2925 70.42) (width 0.25) (layer F.Cu) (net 8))
 (segment (start 139.50001 75.62751) (end 134.754112 70.881612) (width 0.25) (layer F.Cu) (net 8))
 (segment (start 139.50001 84.2536) (end 139.50001 75.62751) (width 0.25) (layer F.Cu) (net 8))
 (segment (start 141.420009 118.299221) (end 118.74923 140.97) (width 0.25) (layer B.Cu) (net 8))
 (segment (start 141.42001 101.93086) (end 141.420009 118.299221) (width 0.25) (layer B.Cu) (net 8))
 (via (at 93.98 140.97) (size 0.8) (drill 0.4) (layers F.Cu B.Cu) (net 8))
 (segment (start 118.74923 140.97) (end 93.98 140.97) (width 0.25) (layer B.Cu) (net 8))
 (segment (start 93.98 140.97) (end 93.98 139.8525) (width 0.25) (layer F.Cu) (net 8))
 (via (at 50.8 71.12) (size 0.8) (drill 0.4) (layers F.Cu B.Cu) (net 8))
 (segment (start 44.994999 76.925001) (end 50.8 71.12) (width 0.25) (layer B.Cu) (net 8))
 (segment (start 44.994999 111.477231) (end 44.994999 76.925001) (width 0.25) (layer B.Cu) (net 8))
 (segment (start 74.487768 140.97) (end 44.994999 111.477231) (width 0.25) (layer B.Cu) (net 8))
 (segment (start 93.98 140.97) (end 74.487768 140.97) (width 0.25) (layer B.Cu) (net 8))
 (segment (start 51.435 70.485) (end 53.8225 70.485) (width 0.25) (layer F.Cu) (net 8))
 (segment (start 50.8 71.12) (end 51.435 70.485) (width 0.25) (layer F.Cu) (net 8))
 (segment (start 138.7375 84.1275) (end 138.7375 81.85) (width 0.25) (layer F.Cu) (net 6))
 (via (at 81.28 142.24) (size 0.8) (drill 0.4) (layers F.Cu B.Cu) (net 6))
 (segment (start 81.28 142.24) (end 81.28 137.9475) (width 0.25) (layer F.Cu) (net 6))
 (segment (start 118.11564 142.24) (end 81.28 142.24) (width 0.25) (layer B.Cu) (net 6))
 (segment (start 143.51 116.84564) (end 118.11564 142.24) (width 0.25) (layer B.Cu) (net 6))
 (segment (start 143.51 101.6) (end 143.51 116.84564) (width 0.25) (layer B.Cu) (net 6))
 (segment (start 44.544989 111.663631) (end 44.544989 74.835011) (width 0.25) (layer B.Cu) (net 6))
 (segment (start 74.396357 141.514999) (end 44.544989 111.663631) (width 0.25) (layer B.Cu) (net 6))
 (segment (start 80.554999 141.514999) (end 74.396357 141.514999) (width 0.25) (layer B.Cu) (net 6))
 (segment (start 81.28 142.24) (end 80.554999 141.514999) (width 0.25) (layer B.Cu) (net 6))
 (via (at 59.69 59.69) (size 0.8) (drill 0.4) (layers F.Cu B.Cu) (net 6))
 (segment (start 44.544989 74.835011) (end 59.69 59.69) (width 0.25) (layer B.Cu) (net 6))
 (segment (start 60.325 59.69) (end 61.038153 60.403153) (width 0.25) (layer F.Cu) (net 6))
 (segment (start 59.69 59.69) (end 60.325 59.69) (width 0.25) (layer F.Cu) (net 6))
 (segment (start 140.949112 93.806612) (end 140.4875 93.345) (width 0.25) (layer F.Cu) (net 4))
 (segment (start 143.6625 96.52) (end 140.949112 93.806612) (width 0.25) (layer F.Cu) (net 4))
 (segment (start 143.960009 117.032041) (end 117.48205 143.51) (width 0.25) (layer B.Cu) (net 4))
 (segment (start 143.96001 101.93086) (end 143.960009 117.032041) (width 0.25) (layer B.Cu) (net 4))
 (segment (start 72.39 143.51) (end 71.12 142.24) (width 0.25) (layer B.Cu) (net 4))
 (via (at 71.12 142.24) (size 0.8) (drill 0.4) (layers F.Cu B.Cu) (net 4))
 (segment (start 117.48205 143.51) (end 72.39 143.51) (width 0.25) (layer B.Cu) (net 4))
 (segment (start 71.12 142.24) (end 71.12 133.5025) (width 0.25) (layer F.Cu) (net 4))
 (via (at 69.85 50.8) (size 0.8) (drill 0.4) (layers F.Cu B.Cu) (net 4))
 (segment (start 43.18 75.126998) (end 67.506998 50.8) (width 0.25) (layer B.Cu) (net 4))
 (segment (start 43.18 114.3) (end 43.18 75.126998) (width 0.25) (layer B.Cu) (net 4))
 (segment (start 67.506998 50.8) (end 69.85 50.8) (width 0.25) (layer B.Cu) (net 4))
 (segment (start 71.12 142.24) (end 43.18 114.3) (width 0.25) (layer B.Cu) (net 4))
 (segment (start 69.85 52.5525) (end 70.485 53.1875) (width 0.25) (layer F.Cu) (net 4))
 (segment (start 69.85 50.8) (end 69.85 52.5525) (width 0.25) (layer F.Cu) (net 4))
 (segment (start 149.86 111.76846) (end 116.84846 144.78) (width 0.25) (layer B.Cu) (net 2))
 (via (at 60.96 134.62) (size 0.8) (drill 0.4) (layers F.Cu B.Cu) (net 2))
 (segment (start 71.12 144.78) (end 60.96 134.62) (width 0.25) (layer B.Cu) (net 2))
 (segment (start 116.84846 144.78) (end 71.12 144.78) (width 0.25) (layer B.Cu) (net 2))
 (segment (start 60.96 126.365) (end 61.038153 126.286847) (width 0.25) (layer F.Cu) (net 2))
 (segment (start 60.96 134.62) (end 60.96 126.365) (width 0.25) (layer F.Cu) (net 2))
 (segment (start 70.680588 46.99) (end 81.28 46.99) (width 0.25) (layer B.Cu) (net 2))
 (segment (start 42.729991 74.940597) (end 70.680588 46.99) (width 0.25) (layer B.Cu) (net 2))
 (via (at 81.28 46.99) (size 0.8) (drill 0.4) (layers F.Cu B.Cu) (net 2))
 (segment (start 42.729991 116.389991) (end 42.729991 74.940597) (width 0.25) (layer B.Cu) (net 2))
 (segment (start 60.96 134.62) (end 42.729991 116.389991) (width 0.25) (layer B.Cu) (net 2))
 (segment (start 81.28 46.99) (end 81.28 48.7425) (width 0.25) (layer F.Cu) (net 2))
 (segment (start 132.5625 118.418806) (end 125.808153 125.173153) (width 0.25) (layer F.Cu) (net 10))
 (segment (start 132.5625 116.205) (end 132.5625 118.418806) (width 0.25) (layer F.Cu) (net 10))
 (segment (start 123.594347 125.173153) (end 116.84 131.9275) (width 0.25) (layer F.Cu) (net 10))
 (segment (start 125.808153 125.173153) (end 123.594347 125.173153) (width 0.25) (layer F.Cu) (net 10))
 (segment (start 110.49 131.9275) (end 106.045 136.3725) (width 0.25) (layer F.Cu) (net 10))
 (segment (start 116.84 131.9275) (end 110.49 131.9275) (width 0.25) (layer F.Cu) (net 10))
 (segment (start 95.885 136.3725) (end 93.98 138.2775) (width 0.25) (layer F.Cu) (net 10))
 (segment (start 106.045 136.3725) (end 95.885 136.3725) (width 0.25) (layer F.Cu) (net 10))
 (segment (start 83.185 138.2775) (end 81.28 136.3725) (width 0.25) (layer F.Cu) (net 10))
 (segment (start 93.98 138.2775) (end 83.185 138.2775) (width 0.25) (layer F.Cu) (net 10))
 (segment (start 75.565 136.3725) (end 71.12 131.9275) (width 0.25) (layer F.Cu) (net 10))
 (segment (start 81.28 136.3725) (end 75.565 136.3725) (width 0.25) (layer F.Cu) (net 10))
 (segment (start 68.906194 131.9275) (end 62.151847 125.173153) (width 0.25) (layer F.Cu) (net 10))
 (segment (start 71.12 131.9275) (end 68.906194 131.9275) (width 0.25) (layer F.Cu) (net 10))
 (segment (start 55.3975 109.855) (end 50.9525 105.41) (width 0.25) (layer F.Cu) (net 11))
 (segment (start 55.3975 116.205) (end 55.3975 109.855) (width 0.25) (layer F.Cu) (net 11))
 (segment (start 50.9525 95.315) (end 49.0475 93.41) (width 0.25) (layer F.Cu) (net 11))
 (segment (start 50.9525 105.41) (end 50.9525 95.315) (width 0.25) (layer F.Cu) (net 11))
 (segment (start 49.0475 83.185) (end 50.3175 81.915) (width 0.25) (layer F.Cu) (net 11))
 (segment (start 49.0475 93.41) (end 49.0475 83.185) (width 0.25) (layer F.Cu) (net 11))
 (segment (start 50.3175 75.565) (end 55.3975 70.485) (width 0.25) (layer F.Cu) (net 11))
 (segment (start 50.3175 81.915) (end 50.3175 75.565) (width 0.25) (layer F.Cu) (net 11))
 (segment (start 55.3975 68.271194) (end 62.151847 61.516847) (width 0.25) (layer F.Cu) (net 11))
 (segment (start 55.3975 70.485) (end 55.3975 68.271194) (width 0.25) (layer F.Cu) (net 11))
 (segment (start 63.730653 61.516847) (end 70.485 54.7625) (width 0.25) (layer F.Cu) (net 11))
 (segment (start 62.151847 61.516847) (end 63.730653 61.516847) (width 0.25) (layer F.Cu) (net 11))
 (segment (start 76.835 54.7625) (end 81.28 50.3175) (width 0.25) (layer F.Cu) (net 11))
 (segment (start 70.485 54.7625) (end 76.835 54.7625) (width 0.25) (layer F.Cu) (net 11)))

